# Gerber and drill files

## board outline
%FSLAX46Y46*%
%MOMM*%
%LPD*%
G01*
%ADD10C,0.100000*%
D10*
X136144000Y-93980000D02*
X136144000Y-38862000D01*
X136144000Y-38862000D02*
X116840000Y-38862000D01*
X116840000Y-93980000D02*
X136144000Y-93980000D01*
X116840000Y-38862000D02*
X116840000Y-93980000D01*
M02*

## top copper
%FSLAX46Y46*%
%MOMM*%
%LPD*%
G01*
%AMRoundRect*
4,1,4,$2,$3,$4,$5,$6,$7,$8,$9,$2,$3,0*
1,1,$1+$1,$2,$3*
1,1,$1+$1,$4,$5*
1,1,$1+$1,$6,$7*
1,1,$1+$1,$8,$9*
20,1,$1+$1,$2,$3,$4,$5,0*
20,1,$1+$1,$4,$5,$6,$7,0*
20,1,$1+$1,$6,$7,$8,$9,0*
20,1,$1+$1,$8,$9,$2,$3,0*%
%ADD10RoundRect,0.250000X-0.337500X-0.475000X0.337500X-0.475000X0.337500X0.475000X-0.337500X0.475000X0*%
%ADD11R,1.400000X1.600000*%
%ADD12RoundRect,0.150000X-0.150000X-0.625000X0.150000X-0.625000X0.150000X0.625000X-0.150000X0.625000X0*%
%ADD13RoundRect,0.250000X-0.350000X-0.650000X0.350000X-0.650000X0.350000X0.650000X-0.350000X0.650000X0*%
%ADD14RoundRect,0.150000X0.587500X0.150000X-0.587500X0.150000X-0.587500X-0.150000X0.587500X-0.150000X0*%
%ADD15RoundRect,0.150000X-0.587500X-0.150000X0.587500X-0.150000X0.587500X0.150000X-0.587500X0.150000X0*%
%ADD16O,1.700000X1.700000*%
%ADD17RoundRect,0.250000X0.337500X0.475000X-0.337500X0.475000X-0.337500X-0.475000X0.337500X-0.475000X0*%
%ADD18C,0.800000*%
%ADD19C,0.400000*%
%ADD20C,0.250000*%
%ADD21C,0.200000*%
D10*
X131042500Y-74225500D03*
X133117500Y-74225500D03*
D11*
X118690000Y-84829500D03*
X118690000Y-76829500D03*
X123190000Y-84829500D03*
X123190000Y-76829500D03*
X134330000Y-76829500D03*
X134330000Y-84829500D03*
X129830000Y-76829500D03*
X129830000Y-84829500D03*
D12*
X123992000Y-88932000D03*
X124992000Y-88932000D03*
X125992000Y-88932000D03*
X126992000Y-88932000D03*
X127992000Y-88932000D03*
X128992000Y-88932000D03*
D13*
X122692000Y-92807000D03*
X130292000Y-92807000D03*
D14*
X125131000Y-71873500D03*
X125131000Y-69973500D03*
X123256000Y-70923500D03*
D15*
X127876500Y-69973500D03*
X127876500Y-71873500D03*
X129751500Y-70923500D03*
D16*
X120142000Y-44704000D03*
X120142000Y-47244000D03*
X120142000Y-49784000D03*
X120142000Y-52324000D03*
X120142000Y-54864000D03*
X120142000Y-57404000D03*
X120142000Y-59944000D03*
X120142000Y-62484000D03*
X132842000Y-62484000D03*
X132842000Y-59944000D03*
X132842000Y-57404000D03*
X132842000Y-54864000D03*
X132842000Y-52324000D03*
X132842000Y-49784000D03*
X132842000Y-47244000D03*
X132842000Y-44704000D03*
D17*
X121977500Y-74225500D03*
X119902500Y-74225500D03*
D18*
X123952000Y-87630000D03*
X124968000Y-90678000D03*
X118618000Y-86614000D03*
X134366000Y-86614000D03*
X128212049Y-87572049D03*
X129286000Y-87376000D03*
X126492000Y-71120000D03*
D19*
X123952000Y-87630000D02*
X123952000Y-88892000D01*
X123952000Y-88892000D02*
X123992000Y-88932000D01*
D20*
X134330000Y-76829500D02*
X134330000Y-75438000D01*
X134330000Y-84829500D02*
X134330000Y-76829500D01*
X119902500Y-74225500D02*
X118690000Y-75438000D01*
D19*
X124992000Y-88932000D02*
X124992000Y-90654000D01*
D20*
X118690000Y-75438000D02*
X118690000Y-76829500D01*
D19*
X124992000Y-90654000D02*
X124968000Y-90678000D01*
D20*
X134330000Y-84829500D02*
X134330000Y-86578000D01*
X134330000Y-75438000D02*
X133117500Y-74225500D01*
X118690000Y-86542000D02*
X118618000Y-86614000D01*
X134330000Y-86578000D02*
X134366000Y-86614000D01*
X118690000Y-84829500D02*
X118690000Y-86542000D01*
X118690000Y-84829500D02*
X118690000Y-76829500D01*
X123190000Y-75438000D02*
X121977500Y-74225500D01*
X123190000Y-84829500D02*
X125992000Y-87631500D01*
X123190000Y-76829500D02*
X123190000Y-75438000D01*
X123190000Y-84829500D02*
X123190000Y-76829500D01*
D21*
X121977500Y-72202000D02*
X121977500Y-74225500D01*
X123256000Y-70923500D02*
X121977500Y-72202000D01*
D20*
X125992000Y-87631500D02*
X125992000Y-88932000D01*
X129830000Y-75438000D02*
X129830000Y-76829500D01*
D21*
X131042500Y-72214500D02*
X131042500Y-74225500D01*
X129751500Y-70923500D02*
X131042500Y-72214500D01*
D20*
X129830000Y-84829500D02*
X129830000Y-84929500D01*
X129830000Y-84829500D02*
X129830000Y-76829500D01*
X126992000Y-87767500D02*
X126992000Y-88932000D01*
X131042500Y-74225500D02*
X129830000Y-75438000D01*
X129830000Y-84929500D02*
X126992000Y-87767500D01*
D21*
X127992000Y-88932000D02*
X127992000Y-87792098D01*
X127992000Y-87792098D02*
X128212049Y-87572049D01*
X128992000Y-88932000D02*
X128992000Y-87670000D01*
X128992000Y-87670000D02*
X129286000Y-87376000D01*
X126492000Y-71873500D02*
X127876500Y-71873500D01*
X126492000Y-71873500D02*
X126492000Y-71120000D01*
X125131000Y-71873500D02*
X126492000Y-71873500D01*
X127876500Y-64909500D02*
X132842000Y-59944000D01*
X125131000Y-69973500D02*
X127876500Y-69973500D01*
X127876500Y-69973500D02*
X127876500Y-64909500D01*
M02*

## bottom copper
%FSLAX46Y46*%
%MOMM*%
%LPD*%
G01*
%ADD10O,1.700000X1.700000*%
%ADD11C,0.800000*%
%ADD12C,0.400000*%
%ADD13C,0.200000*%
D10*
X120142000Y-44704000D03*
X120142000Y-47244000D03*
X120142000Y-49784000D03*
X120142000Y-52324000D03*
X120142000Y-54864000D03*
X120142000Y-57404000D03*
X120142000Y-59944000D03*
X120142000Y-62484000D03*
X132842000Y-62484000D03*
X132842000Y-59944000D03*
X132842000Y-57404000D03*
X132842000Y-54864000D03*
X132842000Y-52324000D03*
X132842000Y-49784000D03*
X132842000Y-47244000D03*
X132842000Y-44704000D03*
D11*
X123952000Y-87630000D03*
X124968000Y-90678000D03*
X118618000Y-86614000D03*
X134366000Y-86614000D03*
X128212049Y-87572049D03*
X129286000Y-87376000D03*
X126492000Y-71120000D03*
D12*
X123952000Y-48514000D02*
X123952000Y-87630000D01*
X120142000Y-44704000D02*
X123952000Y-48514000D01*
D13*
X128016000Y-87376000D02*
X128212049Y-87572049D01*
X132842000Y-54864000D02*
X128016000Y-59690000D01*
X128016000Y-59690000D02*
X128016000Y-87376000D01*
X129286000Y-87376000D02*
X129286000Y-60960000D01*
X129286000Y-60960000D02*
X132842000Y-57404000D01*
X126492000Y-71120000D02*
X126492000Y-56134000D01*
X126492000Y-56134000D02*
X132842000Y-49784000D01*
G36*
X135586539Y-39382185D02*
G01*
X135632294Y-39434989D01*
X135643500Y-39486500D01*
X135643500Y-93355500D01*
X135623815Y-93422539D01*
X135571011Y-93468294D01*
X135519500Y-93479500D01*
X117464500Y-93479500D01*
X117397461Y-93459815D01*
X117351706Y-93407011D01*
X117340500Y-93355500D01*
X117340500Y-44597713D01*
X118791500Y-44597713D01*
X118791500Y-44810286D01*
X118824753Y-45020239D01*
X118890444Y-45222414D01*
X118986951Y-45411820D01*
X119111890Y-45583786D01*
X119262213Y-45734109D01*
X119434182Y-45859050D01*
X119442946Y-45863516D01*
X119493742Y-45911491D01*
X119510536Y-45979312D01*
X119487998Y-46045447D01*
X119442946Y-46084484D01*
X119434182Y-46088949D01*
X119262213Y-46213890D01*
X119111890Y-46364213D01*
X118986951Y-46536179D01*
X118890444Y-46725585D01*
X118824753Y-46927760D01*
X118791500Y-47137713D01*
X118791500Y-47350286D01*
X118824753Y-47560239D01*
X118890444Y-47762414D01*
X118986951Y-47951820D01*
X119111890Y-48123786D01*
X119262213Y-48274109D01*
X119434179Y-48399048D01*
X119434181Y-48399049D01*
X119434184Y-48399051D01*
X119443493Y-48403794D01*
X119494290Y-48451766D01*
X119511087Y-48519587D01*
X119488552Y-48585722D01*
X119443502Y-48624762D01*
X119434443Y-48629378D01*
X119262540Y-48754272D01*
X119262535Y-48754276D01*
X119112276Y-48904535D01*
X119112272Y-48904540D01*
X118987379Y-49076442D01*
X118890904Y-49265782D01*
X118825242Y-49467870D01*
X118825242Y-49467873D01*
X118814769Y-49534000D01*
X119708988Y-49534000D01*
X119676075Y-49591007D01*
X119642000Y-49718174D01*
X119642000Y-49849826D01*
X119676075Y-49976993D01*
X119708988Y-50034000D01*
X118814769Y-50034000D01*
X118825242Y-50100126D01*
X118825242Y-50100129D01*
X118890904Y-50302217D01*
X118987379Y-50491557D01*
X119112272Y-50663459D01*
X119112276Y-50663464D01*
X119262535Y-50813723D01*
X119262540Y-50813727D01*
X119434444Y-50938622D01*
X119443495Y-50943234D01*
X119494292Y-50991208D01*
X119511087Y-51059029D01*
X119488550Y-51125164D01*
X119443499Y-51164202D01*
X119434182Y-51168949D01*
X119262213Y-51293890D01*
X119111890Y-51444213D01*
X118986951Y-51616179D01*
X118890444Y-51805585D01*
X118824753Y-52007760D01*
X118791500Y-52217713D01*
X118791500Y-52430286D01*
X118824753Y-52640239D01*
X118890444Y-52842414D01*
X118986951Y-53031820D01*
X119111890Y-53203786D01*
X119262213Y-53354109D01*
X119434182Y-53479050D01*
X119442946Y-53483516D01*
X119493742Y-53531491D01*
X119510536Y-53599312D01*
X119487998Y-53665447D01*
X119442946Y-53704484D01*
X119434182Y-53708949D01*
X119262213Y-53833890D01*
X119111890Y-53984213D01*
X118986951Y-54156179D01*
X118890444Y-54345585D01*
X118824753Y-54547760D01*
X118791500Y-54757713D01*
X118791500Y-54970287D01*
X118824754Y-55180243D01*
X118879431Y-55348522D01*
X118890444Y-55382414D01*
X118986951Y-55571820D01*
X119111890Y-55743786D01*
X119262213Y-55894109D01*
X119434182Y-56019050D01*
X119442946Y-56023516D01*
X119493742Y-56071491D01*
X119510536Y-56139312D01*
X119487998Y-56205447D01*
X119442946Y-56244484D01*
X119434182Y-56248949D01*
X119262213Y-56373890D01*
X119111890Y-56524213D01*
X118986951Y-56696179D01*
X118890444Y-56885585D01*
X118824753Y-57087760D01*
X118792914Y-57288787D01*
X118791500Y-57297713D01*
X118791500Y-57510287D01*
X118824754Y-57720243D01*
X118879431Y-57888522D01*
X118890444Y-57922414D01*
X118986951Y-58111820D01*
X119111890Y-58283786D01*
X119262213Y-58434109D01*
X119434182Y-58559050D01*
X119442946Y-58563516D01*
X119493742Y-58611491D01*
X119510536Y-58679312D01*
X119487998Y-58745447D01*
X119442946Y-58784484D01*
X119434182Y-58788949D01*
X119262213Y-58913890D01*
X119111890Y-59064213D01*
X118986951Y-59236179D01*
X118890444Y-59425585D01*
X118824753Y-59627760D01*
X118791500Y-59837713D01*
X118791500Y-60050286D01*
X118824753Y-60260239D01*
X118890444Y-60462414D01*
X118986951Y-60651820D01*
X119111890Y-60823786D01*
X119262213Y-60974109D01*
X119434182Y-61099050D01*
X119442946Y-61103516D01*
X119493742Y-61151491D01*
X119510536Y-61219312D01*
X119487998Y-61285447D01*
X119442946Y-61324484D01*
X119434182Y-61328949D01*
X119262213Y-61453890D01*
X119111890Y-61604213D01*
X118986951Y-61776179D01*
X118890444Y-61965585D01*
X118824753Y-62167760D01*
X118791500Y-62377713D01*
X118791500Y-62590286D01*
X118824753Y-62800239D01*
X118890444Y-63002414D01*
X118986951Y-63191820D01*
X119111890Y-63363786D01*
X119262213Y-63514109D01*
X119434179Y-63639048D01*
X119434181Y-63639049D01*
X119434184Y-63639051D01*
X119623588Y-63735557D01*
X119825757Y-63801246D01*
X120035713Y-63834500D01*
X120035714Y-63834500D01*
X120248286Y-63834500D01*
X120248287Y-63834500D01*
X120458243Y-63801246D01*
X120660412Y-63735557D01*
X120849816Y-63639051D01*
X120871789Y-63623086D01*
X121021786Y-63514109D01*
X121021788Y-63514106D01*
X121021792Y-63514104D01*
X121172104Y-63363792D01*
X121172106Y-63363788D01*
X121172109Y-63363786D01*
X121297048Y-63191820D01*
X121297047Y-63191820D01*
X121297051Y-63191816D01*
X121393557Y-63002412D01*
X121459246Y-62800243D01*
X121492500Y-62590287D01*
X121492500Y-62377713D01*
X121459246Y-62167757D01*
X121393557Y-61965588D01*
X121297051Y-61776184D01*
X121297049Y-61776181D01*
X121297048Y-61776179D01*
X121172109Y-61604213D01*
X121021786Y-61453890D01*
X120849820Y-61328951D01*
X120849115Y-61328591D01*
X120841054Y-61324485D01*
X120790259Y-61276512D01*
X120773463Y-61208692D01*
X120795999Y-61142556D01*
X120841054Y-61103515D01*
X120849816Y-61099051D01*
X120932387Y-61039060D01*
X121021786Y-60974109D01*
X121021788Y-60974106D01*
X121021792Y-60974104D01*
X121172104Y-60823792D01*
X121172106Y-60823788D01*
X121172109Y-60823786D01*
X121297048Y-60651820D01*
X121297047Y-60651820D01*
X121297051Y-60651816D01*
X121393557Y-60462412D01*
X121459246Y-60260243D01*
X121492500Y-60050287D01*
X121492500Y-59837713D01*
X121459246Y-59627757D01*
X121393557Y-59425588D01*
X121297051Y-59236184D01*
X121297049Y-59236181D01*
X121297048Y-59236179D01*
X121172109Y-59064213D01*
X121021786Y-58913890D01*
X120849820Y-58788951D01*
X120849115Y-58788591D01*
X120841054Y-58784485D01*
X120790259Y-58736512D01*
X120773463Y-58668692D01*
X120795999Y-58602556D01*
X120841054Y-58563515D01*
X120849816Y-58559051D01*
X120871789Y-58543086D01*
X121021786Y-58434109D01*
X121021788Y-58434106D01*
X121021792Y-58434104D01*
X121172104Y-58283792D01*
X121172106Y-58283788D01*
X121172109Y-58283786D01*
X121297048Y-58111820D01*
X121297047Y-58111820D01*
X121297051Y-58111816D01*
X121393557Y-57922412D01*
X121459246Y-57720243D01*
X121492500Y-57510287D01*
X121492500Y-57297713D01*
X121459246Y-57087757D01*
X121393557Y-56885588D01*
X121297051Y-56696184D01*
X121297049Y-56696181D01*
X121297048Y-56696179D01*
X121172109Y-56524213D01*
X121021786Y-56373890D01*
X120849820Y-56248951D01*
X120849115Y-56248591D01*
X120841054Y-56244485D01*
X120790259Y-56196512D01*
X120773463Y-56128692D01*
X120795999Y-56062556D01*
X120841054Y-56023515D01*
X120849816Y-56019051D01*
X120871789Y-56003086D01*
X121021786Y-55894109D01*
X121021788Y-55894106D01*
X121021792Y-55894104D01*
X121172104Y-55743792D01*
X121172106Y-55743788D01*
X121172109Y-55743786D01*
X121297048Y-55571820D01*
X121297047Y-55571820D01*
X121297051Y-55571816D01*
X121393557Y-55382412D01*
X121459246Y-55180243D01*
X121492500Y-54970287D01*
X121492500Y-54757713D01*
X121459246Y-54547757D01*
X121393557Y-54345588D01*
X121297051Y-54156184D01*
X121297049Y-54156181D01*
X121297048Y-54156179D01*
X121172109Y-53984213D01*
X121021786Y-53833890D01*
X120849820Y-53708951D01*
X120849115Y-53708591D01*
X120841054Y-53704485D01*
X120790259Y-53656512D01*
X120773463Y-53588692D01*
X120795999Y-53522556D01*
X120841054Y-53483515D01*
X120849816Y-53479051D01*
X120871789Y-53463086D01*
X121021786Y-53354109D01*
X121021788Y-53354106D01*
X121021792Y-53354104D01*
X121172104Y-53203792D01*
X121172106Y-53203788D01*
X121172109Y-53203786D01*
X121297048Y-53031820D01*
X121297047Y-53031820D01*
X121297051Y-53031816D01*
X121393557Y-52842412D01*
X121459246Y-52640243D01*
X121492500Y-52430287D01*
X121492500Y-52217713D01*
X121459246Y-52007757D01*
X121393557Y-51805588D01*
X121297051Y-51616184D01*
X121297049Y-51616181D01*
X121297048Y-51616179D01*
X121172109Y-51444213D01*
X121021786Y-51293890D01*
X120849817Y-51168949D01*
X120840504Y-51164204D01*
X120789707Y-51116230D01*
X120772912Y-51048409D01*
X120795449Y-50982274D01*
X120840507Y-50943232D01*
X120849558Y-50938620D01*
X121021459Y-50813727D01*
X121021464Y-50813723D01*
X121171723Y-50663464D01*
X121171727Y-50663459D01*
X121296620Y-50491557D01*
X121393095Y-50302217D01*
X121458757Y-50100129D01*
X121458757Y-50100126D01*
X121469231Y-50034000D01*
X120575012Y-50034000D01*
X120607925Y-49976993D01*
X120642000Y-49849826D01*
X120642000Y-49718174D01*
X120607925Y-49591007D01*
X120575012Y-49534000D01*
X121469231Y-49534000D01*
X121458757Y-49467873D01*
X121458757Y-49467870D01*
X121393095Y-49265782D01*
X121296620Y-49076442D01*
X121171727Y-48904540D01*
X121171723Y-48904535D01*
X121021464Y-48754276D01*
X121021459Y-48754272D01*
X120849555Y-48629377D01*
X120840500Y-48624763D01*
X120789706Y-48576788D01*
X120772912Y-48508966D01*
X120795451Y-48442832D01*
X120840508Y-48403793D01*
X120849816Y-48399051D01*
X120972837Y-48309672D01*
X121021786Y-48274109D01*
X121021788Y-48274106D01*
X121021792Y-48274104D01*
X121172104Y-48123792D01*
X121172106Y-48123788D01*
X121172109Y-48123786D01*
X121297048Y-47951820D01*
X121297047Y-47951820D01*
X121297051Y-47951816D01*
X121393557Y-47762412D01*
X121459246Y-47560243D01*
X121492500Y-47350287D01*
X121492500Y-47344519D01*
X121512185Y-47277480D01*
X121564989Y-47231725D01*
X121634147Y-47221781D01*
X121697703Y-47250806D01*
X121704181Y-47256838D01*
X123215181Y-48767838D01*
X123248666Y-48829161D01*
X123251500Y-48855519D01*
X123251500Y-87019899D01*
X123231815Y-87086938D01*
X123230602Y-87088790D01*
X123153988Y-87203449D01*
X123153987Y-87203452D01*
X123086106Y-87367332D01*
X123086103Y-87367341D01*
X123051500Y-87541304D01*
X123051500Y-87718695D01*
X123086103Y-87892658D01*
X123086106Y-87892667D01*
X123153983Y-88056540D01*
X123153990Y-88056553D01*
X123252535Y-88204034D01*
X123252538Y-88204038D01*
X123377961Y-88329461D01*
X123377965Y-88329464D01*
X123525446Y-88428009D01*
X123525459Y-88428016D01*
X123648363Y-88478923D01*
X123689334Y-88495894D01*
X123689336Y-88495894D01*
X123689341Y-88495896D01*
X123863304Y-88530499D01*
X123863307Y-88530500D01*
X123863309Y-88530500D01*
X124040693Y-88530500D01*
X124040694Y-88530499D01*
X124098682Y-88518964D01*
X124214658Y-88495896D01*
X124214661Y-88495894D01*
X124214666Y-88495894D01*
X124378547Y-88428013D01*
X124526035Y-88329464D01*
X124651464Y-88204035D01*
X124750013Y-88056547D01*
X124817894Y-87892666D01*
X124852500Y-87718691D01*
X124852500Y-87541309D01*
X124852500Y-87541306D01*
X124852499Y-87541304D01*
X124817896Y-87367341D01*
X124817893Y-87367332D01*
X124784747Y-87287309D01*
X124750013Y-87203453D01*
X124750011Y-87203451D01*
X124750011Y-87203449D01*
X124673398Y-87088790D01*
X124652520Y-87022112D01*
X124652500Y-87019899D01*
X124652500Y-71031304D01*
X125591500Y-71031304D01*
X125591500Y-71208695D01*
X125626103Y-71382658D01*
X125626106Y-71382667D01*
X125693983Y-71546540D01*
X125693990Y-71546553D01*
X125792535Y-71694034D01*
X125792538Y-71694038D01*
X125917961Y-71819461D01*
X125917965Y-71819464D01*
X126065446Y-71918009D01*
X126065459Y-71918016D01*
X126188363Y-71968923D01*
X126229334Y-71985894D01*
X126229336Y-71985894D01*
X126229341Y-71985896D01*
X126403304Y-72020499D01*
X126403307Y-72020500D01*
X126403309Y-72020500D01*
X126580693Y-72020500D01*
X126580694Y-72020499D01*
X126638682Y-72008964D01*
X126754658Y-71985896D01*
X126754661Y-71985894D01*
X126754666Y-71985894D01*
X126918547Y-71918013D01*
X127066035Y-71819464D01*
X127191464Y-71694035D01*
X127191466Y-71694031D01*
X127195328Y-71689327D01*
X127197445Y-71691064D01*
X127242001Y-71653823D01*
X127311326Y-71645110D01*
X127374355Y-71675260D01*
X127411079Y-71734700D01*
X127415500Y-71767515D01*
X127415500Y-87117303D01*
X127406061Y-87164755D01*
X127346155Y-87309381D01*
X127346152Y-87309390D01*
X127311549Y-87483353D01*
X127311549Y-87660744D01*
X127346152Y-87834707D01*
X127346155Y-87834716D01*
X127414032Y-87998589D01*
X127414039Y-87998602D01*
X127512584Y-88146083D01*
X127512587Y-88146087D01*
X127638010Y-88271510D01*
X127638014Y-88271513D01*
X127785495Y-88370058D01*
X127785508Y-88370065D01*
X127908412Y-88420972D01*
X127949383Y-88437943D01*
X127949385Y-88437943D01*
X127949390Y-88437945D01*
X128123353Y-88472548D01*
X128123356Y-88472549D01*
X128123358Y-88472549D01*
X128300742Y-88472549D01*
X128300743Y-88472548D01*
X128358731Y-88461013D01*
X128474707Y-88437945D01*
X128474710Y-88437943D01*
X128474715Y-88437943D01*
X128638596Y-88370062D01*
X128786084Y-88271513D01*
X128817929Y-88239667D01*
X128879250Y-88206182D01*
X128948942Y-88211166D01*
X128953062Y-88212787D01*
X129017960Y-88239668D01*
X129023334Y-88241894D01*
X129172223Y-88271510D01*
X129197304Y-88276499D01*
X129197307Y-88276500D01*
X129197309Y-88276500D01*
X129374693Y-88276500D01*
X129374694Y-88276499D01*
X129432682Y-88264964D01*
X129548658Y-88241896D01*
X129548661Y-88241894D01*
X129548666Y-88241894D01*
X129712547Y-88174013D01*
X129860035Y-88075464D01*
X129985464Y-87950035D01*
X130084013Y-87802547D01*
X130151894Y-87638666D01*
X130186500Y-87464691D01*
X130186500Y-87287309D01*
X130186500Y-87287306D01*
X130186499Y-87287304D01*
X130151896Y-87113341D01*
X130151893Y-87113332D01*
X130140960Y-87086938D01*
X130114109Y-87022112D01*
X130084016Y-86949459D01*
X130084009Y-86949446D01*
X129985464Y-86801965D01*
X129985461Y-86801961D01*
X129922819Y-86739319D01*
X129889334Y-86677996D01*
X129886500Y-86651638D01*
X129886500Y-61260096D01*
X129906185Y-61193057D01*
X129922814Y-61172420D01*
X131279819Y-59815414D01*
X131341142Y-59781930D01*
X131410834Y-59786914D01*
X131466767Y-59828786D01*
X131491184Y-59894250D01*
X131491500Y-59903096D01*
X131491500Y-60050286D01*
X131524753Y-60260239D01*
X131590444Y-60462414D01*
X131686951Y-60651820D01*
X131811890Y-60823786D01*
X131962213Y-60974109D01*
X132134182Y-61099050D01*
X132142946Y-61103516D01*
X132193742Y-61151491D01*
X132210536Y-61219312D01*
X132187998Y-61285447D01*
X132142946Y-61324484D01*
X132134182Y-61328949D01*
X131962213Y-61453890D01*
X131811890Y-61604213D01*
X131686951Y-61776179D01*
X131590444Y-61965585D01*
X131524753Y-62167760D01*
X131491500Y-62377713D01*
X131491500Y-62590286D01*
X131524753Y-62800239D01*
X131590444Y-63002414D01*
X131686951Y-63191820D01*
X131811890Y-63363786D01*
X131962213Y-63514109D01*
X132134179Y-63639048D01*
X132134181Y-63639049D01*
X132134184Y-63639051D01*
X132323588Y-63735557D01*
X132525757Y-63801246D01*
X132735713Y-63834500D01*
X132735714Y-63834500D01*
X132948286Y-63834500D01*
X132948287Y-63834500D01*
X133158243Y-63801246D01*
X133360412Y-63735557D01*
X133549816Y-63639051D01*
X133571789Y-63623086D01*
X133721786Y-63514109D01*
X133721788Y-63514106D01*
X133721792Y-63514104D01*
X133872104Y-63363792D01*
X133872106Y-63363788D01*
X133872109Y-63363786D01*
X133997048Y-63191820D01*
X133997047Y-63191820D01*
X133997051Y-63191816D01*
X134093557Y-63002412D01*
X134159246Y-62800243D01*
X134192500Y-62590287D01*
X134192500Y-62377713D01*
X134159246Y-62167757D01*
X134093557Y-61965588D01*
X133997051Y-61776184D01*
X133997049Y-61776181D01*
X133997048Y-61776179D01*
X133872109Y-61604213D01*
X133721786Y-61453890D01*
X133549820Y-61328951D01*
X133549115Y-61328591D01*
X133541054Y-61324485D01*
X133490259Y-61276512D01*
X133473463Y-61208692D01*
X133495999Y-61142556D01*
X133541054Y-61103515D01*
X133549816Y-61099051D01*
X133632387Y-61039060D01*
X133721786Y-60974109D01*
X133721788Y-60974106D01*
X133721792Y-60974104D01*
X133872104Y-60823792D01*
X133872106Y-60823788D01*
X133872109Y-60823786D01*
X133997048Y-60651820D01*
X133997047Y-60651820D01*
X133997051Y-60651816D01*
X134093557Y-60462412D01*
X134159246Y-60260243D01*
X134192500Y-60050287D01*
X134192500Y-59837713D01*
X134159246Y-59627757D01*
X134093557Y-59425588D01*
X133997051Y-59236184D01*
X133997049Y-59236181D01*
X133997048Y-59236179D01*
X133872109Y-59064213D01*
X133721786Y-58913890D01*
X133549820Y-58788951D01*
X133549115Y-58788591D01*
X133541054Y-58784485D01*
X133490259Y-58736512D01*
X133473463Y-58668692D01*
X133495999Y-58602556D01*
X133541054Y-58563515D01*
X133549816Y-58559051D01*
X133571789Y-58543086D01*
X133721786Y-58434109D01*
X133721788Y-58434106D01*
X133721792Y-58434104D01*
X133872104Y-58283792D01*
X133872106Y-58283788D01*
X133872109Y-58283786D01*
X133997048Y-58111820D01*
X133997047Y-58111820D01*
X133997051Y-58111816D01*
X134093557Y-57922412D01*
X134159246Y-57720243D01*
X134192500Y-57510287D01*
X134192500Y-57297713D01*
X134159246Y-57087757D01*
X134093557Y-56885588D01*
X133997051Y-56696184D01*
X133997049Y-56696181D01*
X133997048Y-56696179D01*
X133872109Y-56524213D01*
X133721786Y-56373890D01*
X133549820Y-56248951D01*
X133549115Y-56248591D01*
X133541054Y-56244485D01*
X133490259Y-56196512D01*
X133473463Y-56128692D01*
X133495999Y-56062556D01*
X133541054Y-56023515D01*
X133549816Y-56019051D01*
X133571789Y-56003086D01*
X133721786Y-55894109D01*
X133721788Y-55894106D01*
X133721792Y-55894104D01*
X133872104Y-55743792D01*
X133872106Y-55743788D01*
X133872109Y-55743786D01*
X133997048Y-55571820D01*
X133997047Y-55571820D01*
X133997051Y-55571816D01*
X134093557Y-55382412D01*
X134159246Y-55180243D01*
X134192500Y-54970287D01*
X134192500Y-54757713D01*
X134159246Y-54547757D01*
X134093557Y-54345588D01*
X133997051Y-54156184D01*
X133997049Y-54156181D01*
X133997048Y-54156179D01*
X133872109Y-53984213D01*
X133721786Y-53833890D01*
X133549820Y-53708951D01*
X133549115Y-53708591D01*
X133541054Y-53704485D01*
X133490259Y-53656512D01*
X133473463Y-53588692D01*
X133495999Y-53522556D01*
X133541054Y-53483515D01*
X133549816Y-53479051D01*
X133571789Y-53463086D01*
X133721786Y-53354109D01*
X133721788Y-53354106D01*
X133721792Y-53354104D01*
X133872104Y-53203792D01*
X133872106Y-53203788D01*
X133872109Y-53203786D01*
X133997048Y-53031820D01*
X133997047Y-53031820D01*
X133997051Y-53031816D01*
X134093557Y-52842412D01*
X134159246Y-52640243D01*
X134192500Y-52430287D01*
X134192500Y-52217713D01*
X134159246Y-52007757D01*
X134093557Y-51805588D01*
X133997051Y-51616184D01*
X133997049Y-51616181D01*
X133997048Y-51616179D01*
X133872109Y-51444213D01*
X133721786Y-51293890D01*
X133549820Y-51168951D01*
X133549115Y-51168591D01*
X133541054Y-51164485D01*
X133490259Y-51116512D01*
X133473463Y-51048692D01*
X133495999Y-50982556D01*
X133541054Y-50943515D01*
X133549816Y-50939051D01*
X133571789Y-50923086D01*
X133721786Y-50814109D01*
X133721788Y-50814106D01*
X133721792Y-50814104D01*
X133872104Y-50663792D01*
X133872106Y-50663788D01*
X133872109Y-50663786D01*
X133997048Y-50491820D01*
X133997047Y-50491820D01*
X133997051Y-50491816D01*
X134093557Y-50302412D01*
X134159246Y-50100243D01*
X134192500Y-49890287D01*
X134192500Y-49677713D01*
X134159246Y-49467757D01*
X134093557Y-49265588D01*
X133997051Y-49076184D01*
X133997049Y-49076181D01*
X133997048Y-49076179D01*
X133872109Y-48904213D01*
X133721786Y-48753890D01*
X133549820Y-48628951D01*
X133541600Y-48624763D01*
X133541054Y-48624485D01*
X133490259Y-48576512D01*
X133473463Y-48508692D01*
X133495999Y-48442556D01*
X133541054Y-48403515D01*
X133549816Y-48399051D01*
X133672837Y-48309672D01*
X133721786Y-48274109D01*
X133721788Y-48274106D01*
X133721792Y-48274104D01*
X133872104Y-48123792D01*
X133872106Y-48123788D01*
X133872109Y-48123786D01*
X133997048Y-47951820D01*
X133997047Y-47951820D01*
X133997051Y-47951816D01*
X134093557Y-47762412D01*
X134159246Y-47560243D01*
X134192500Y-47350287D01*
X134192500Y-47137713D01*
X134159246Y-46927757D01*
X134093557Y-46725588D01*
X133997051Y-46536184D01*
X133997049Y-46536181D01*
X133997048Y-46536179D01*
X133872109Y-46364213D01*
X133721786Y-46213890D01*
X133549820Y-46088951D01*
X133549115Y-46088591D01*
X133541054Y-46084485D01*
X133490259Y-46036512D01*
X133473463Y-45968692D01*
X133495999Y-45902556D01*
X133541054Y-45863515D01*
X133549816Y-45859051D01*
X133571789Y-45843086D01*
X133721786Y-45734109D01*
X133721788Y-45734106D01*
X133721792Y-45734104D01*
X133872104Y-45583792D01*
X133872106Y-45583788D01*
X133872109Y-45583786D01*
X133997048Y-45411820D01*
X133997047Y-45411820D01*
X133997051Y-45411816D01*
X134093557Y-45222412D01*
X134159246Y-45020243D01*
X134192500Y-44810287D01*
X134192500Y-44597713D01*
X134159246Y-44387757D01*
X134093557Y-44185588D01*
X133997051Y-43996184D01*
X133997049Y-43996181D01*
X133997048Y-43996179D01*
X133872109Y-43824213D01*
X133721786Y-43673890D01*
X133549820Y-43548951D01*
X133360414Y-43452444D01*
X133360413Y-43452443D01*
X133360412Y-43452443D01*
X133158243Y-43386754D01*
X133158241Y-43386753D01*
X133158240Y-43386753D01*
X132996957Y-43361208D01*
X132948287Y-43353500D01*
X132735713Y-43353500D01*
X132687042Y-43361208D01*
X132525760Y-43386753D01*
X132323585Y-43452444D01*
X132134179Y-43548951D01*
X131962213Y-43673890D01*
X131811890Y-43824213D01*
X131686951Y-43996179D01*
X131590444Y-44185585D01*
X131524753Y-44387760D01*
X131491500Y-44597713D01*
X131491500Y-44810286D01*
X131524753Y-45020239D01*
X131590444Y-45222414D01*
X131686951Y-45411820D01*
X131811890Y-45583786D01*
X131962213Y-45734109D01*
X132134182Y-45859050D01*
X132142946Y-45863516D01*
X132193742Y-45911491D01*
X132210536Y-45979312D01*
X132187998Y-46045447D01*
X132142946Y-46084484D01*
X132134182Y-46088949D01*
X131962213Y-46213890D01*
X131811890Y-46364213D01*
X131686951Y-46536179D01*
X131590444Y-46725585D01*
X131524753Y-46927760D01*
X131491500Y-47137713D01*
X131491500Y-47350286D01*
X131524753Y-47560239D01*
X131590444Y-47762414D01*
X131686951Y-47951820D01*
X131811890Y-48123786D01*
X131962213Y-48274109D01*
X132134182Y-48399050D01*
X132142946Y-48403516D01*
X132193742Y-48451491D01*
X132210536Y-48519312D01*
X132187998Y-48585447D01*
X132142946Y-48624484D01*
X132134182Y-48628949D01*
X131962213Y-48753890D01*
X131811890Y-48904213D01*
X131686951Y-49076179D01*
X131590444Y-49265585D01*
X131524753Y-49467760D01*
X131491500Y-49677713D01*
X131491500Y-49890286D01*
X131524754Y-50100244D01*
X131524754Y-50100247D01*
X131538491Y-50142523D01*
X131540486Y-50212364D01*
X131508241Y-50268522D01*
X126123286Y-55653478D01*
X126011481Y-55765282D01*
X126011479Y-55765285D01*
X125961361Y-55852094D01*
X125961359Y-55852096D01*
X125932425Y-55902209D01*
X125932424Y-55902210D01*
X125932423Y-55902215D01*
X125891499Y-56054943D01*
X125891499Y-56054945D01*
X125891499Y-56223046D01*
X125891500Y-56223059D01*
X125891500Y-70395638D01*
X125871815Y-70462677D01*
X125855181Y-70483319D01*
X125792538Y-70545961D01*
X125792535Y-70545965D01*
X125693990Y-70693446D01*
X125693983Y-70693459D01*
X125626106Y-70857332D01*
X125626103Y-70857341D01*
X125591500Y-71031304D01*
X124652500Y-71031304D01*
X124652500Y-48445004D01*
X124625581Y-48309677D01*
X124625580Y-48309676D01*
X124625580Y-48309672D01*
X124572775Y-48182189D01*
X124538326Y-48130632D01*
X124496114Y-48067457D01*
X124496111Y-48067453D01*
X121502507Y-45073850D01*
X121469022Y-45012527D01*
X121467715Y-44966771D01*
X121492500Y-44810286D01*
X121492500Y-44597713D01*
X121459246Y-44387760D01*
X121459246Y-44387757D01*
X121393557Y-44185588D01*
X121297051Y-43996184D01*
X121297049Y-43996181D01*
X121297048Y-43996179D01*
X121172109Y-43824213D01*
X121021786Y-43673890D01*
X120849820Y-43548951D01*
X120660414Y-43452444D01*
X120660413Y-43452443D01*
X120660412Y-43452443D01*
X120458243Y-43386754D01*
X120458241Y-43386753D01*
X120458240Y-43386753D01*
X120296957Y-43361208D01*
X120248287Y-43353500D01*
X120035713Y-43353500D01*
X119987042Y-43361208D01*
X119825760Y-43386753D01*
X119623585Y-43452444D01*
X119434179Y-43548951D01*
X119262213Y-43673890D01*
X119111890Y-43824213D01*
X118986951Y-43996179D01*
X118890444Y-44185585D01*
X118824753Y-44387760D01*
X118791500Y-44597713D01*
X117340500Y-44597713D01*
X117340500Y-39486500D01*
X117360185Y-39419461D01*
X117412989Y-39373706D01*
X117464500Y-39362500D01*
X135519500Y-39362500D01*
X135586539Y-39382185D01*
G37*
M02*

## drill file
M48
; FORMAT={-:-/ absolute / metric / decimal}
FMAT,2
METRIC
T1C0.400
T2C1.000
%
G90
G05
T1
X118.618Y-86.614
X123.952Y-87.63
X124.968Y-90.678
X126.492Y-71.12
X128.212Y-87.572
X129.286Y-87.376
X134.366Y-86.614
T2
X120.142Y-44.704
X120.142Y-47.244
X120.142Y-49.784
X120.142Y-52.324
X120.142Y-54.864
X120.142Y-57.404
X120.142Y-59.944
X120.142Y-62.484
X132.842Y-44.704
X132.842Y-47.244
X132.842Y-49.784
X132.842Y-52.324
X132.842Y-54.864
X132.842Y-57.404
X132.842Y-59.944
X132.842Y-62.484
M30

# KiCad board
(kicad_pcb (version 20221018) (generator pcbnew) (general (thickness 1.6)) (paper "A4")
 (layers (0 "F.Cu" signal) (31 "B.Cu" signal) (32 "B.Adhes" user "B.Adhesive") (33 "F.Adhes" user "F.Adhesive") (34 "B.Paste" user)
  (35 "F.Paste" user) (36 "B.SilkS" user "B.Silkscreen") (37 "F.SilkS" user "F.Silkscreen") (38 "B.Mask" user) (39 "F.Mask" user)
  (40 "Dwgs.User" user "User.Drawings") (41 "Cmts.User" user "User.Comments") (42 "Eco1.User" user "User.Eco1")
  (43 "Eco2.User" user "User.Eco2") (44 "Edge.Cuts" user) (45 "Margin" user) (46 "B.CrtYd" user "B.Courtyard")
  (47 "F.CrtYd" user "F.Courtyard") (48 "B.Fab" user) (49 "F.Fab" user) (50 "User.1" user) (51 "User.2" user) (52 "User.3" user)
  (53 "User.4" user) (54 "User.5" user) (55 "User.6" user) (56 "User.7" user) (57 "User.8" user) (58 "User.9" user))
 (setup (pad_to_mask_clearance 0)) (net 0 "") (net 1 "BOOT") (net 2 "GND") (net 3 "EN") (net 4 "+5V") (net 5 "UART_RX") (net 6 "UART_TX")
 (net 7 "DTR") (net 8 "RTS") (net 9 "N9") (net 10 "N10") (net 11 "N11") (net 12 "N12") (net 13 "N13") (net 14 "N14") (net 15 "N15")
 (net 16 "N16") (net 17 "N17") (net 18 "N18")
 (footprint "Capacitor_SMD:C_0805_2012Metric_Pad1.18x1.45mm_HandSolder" (layer "F.Cu") (at 132.08 74.2255)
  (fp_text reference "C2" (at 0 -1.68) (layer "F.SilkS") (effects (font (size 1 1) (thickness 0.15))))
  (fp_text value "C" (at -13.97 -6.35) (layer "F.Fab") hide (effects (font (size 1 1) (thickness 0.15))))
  (pad "1" smd roundrect (at -1.0375 0) (size 1.175 1.45) (layers "F.Cu" "F.Paste" "F.Mask") (roundrect_rratio 0.2127659574) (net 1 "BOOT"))
  (pad "2" smd roundrect (at 1.0375 0) (size 1.175 1.45) (layers "F.Cu" "F.Paste" "F.Mask") (roundrect_rratio 0.2127659574) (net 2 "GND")))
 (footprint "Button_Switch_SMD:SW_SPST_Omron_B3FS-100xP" (layer "F.Cu") (at 120.94 80.8295 90)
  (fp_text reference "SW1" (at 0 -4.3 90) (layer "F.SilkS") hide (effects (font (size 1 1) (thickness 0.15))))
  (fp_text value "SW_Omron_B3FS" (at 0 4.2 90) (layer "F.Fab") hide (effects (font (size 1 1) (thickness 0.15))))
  (pad "1" smd rect (at -4 -2.25 270) (size 1.6 1.4) (layers "F.Cu" "F.Paste" "F.Mask") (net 2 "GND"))
  (pad "1" smd rect (at 4 -2.25 270) (size 1.6 1.4) (layers "F.Cu" "F.Paste" "F.Mask") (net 2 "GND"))
  (pad "2" smd rect (at -4 2.25 270) (size 1.6 1.4) (layers "F.Cu" "F.Paste" "F.Mask") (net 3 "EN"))
  (pad "2" smd rect (at 4 2.25 270) (size 1.6 1.4) (layers "F.Cu" "F.Paste" "F.Mask") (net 3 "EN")))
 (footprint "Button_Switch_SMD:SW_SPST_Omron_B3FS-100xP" (layer "F.Cu") (at 132.08 80.8295 -90)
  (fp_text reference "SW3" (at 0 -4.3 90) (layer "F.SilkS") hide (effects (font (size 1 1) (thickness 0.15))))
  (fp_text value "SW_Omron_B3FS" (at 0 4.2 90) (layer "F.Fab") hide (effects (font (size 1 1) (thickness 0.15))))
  (pad "1" smd rect (at -4 -2.25 90) (size 1.6 1.4) (layers "F.Cu" "F.Paste" "F.Mask") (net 2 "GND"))
  (pad "1" smd rect (at 4 -2.25 90) (size 1.6 1.4) (layers "F.Cu" "F.Paste" "F.Mask") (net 2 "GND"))
  (pad "2" smd rect (at -4 2.25 90) (size 1.6 1.4) (layers "F.Cu" "F.Paste" "F.Mask") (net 1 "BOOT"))
  (pad "2" smd rect (at 4 2.25 90) (size 1.6 1.4) (layers "F.Cu" "F.Paste" "F.Mask") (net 1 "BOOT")))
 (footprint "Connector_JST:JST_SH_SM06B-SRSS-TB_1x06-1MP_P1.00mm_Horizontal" (layer "F.Cu") (at 126.492 90.932)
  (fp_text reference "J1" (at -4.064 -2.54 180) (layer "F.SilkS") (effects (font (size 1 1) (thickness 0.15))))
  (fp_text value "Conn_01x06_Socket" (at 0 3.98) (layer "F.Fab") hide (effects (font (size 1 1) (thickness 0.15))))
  (pad "1" smd roundrect (at -2.5 -2) (size 0.6 1.55) (layers "F.Cu" "F.Paste" "F.Mask") (roundrect_rratio 0.25) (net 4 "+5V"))
  (pad "2" smd roundrect (at -1.5 -2) (size 0.6 1.55) (layers "F.Cu" "F.Paste" "F.Mask") (roundrect_rratio 0.25) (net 2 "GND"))
  (pad "3" smd roundrect (at -0.5 -2) (size 0.6 1.55) (layers "F.Cu" "F.Paste" "F.Mask") (roundrect_rratio 0.25) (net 3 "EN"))
  (pad "4" smd roundrect (at 0.5 -2) (size 0.6 1.55) (layers "F.Cu" "F.Paste" "F.Mask") (roundrect_rratio 0.25) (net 1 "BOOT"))
  (pad "5" smd roundrect (at 1.5 -2) (size 0.6 1.55) (layers "F.Cu" "F.Paste" "F.Mask") (roundrect_rratio 0.25) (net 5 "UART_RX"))
  (pad "6" smd roundrect (at 2.5 -2) (size 0.6 1.55) (layers "F.Cu" "F.Paste" "F.Mask") (roundrect_rratio 0.25) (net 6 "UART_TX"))
  (pad "MP" smd roundrect (at -3.8 1.875) (size 1.2 1.8) (layers "F.Cu" "F.Paste" "F.Mask") (roundrect_rratio 0.2083333333))
  (pad "MP" smd roundrect (at 3.8 1.875) (size 1.2 1.8) (layers "F.Cu" "F.Paste" "F.Mask") (roundrect_rratio 0.2083333333)))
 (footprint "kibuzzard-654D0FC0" (layer "F.Cu") (at 120.904 86.868)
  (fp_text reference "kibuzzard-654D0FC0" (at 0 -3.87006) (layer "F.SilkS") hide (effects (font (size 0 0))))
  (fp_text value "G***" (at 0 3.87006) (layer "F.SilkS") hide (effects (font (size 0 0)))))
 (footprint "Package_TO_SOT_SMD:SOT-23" (layer "F.Cu") (at 124.1935 70.9235 180)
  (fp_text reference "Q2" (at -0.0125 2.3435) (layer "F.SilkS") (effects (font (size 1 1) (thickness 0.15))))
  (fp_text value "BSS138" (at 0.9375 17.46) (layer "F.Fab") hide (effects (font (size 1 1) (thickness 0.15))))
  (pad "1" smd roundrect (at -0.9375 -0.95 180) (size 1.475 0.6) (layers "F.Cu" "F.Paste" "F.Mask") (roundrect_rratio 0.25) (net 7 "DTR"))
  (pad "2" smd roundrect (at -0.9375 0.95 180) (size 1.475 0.6) (layers "F.Cu" "F.Paste" "F.Mask") (roundrect_rratio 0.25) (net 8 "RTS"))
  (pad "3" smd roundrect (at 0.9375 0 180) (size 1.475 0.6) (layers "F.Cu" "F.Paste" "F.Mask") (roundrect_rratio 0.25) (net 3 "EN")))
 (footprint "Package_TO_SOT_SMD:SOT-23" (layer "F.Cu") (at 128.814 70.9235)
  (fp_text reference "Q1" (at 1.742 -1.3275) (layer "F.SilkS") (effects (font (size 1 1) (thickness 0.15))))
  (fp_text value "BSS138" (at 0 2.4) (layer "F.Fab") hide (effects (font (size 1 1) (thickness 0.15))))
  (pad "1" smd roundrect (at -0.9375 -0.95) (size 1.475 0.6) (layers "F.Cu" "F.Paste" "F.Mask") (roundrect_rratio 0.25) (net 8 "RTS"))
  (pad "2" smd roundrect (at -0.9375 0.95) (size 1.475 0.6) (layers "F.Cu" "F.Paste" "F.Mask") (roundrect_rratio 0.25) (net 7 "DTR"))
  (pad "3" smd roundrect (at 0.9375 0) (size 1.475 0.6) (layers "F.Cu" "F.Paste" "F.Mask") (roundrect_rratio 0.25) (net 1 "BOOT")))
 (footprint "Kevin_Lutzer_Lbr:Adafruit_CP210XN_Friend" (layer "F.Cu") (at 126.492 53.594)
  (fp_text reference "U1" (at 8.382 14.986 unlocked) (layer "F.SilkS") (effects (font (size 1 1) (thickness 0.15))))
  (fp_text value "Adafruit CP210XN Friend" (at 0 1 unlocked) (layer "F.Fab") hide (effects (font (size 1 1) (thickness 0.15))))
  (pad "1" thru_hole oval (at -6.35 -8.89) (size 1.7 1.7) (drill 1) (layers "*.Cu" "*.Mask") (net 4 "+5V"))
  (pad "2" thru_hole oval (at -6.35 -6.35) (size 1.7 1.7) (drill 1) (layers "*.Cu" "*.Mask") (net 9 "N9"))
  (pad "3" thru_hole oval (at -6.35 -3.81) (size 1.7 1.7) (drill 1) (layers "*.Cu" "*.Mask") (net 2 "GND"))
  (pad "4" thru_hole oval (at -6.35 -1.27) (size 1.7 1.7) (drill 1) (layers "*.Cu" "*.Mask") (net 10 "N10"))
  (pad "5" thru_hole oval (at -6.35 1.27) (size 1.7 1.7) (drill 1) (layers "*.Cu" "*.Mask") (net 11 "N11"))
  (pad "6" thru_hole oval (at -6.35 3.81) (size 1.7 1.7) (drill 1) (layers "*.Cu" "*.Mask") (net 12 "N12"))
  (pad "7" thru_hole oval (at -6.35 6.35) (size 1.7 1.7) (drill 1) (layers "*.Cu" "*.Mask") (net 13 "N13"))
  (pad "8" thru_hole oval (at -6.35 8.89) (size 1.7 1.7) (drill 1) (layers "*.Cu" "*.Mask") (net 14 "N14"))
  (pad "9" thru_hole oval (at 6.35 8.89) (size 1.7 1.7) (drill 1) (layers "*.Cu" "*.Mask") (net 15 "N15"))
  (pad "10" thru_hole oval (at 6.35 6.35) (size 1.7 1.7) (drill 1) (layers "*.Cu" "*.Mask") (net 8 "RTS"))
  (pad "11" thru_hole oval (at 6.35 3.81) (size 1.7 1.7) (drill 1) (layers "*.Cu" "*.Mask") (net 6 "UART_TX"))
  (pad "12" thru_hole oval (at 6.35 1.27) (size 1.7 1.7) (drill 1) (layers "*.Cu" "*.Mask") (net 5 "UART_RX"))
  (pad "13" thru_hole oval (at 6.35 -1.27) (size 1.7 1.7) (drill 1) (layers "*.Cu" "*.Mask") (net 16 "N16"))
  (pad "14" thru_hole oval (at 6.35 -3.81) (size 1.7 1.7) (drill 1) (layers "*.Cu" "*.Mask") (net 7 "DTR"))
  (pad "15" thru_hole oval (at 6.35 -6.35) (size 1.7 1.7) (drill 1) (layers "*.Cu" "*.Mask") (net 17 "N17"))
  (pad "16" thru_hole oval (at 6.35 -8.89) (size 1.7 1.7) (drill 1) (layers "*.Cu" "*.Mask") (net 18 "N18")))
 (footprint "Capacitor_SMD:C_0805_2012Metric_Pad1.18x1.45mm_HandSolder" (layer "F.Cu") (at 120.94 74.2255 180)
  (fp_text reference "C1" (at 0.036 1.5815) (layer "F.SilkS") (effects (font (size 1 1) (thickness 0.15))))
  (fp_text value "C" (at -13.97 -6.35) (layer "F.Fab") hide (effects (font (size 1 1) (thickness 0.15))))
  (pad "1" smd roundrect (at -1.0375 0 180) (size 1.175 1.45) (layers "F.Cu" "F.Paste" "F.Mask") (roundrect_rratio 0.2127659574)
   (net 3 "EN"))
  (pad "2" smd roundrect (at 1.0375 0 180) (size 1.175 1.45) (layers "F.Cu" "F.Paste" "F.Mask") (roundrect_rratio 0.2127659574)
   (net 2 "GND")))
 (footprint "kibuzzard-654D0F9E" (layer "F.Cu") (at 132.08 86.868)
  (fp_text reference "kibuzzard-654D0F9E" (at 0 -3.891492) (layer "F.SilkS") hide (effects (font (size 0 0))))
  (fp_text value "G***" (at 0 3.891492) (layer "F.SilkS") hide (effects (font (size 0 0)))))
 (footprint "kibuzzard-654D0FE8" (layer "B.Cu") (at 118.364 73.66 -90)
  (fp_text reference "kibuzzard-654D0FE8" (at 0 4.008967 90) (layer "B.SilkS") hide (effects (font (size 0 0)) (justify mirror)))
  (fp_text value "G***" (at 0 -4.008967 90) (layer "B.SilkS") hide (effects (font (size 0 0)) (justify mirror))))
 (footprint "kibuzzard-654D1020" (layer "B.Cu") (at 120.396 70.104 -90)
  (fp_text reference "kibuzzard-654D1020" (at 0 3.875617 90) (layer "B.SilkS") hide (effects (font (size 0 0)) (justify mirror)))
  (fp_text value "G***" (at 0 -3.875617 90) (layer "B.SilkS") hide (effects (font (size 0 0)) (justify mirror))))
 (gr_line (start 136.144 93.98) (end 136.144 38.862) (stroke (width 0.1) (type default)) (layer "Edge.Cuts"))
 (gr_line (start 136.144 38.862) (end 116.84 38.862) (stroke (width 0.1) (type default)) (layer "Edge.Cuts"))
 (gr_line (start 116.84 93.98) (end 136.144 93.98) (stroke (width 0.1) (type default)) (layer "Edge.Cuts"))
 (gr_line (start 116.84 38.862) (end 116.84 93.98) (stroke (width 0.1) (type default)) (layer "Edge.Cuts"))
 (segment (start 123.952 87.63) (end 123.952 88.892) (width 0.4) (layer "F.Cu") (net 4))
 (segment (start 123.952 88.892) (end 123.992 88.932) (width 0.4) (layer "F.Cu") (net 4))
 (via (at 123.952 87.63) (size 0.8) (drill 0.4) (layers "F.Cu" "B.Cu") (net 4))
 (segment (start 123.952 48.514) (end 123.952 87.63) (width 0.4) (layer "B.Cu") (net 4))
 (segment (start 120.142 44.704) (end 123.952 48.514) (width 0.4) (layer "B.Cu") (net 4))
 (segment (start 134.33 76.8295) (end 134.33 75.438) (width 0.25) (layer "F.Cu") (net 2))
 (segment (start 134.33 84.8295) (end 134.33 76.8295) (width 0.25) (layer "F.Cu") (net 2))
 (segment (start 119.9025 74.2255) (end 118.69 75.438) (width 0.25) (layer "F.Cu") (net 2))
 (segment (start 124.992 88.932) (end 124.992 90.654) (width 0.4) (layer "F.Cu") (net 2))
 (segment (start 118.69 75.438) (end 118.69 76.8295) (width 0.25) (layer "F.Cu") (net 2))
 (segment (start 124.992 90.654) (end 124.968 90.678) (width 0.4) (layer "F.Cu") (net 2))
 (segment (start 134.33 84.8295) (end 134.33 86.578) (width 0.25) (layer "F.Cu") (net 2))
 (segment (start 134.33 75.438) (end 133.1175 74.2255) (width 0.25) (layer "F.Cu") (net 2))
 (segment (start 118.69 86.542) (end 118.618 86.614) (width 0.25) (layer "F.Cu") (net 2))
 (segment (start 134.33 86.578) (end 134.366 86.614) (width 0.25) (layer "F.Cu") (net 2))
 (segment (start 118.69 84.8295) (end 118.69 86.542) (width 0.25) (layer "F.Cu") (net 2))
 (segment (start 118.69 84.8295) (end 118.69 76.8295) (width 0.25) (layer "F.Cu") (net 2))
 (via (at 124.968 90.678) (size 0.8) (drill 0.4) (layers "F.Cu" "B.Cu") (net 2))
 (via (at 118.618 86.614) (size 0.8) (drill 0.4) (layers "F.Cu" "B.Cu") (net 2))
 (via (at 134.366 86.614) (size 0.8) (drill 0.4) (layers "F.Cu" "B.Cu") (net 2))
 (segment (start 123.19 75.438) (end 121.9775 74.2255) (width 0.25) (layer "F.Cu") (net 3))
 (segment (start 123.19 84.8295) (end 125.992 87.6315) (width 0.25) (layer "F.Cu") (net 3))
 (segment (start 123.19 76.8295) (end 123.19 75.438) (width 0.25) (layer "F.Cu") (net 3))
 (segment (start 123.19 84.8295) (end 123.19 76.8295) (width 0.25) (layer "F.Cu") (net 3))
 (segment (start 121.9775 72.202) (end 121.9775 74.2255) (width 0.2) (layer "F.Cu") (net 3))
 (segment (start 123.256 70.9235) (end 121.9775 72.202) (width 0.2) (layer "F.Cu") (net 3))
 (segment (start 125.992 87.6315) (end 125.992 88.932) (width 0.25) (layer "F.Cu") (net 3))
 (segment (start 129.83 75.438) (end 129.83 76.8295) (width 0.25) (layer "F.Cu") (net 1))
 (segment (start 131.0425 72.2145) (end 131.0425 74.2255) (width 0.2) (layer "F.Cu") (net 1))
 (segment (start 129.7515 70.9235) (end 131.0425 72.2145) (width 0.2) (layer "F.Cu") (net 1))
 (segment (start 129.83 84.8295) (end 129.83 84.9295) (width 0.25) (layer "F.Cu") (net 1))
 (segment (start 129.83 84.8295) (end 129.83 76.8295) (width 0.25) (layer "F.Cu") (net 1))
 (segment (start 126.992 87.7675) (end 126.992 88.932) (width 0.25) (layer "F.Cu") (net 1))
 (segment (start 131.0425 74.2255) (end 129.83 75.438) (width 0.25) (layer "F.Cu") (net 1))
 (segment (start 129.83 84.9295) (end 126.992 87.7675) (width 0.25) (layer "F.Cu") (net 1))
 (segment (start 127.992 88.932) (end 127.992 87.792098) (width 0.2) (layer "F.Cu") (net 5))
 (segment (start 127.992 87.792098) (end 128.212049 87.572049) (width 0.2) (layer "F.Cu") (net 5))
 (via (at 128.212049 87.572049) (size 0.8) (drill 0.4) (layers "F.Cu" "B.Cu") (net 5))
 (segment (start 128.016 87.376) (end 128.212049 87.572049) (width 0.2) (layer "B.Cu") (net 5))
 (segment (start 132.842 54.864) (end 128.016 59.69) (width 0.2) (layer "B.Cu") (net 5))
 (segment (start 128.016 59.69) (end 128.016 87.376) (width 0.2) (layer "B.Cu") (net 5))
 (segment (start 128.992 88.932) (end 128.992 87.67) (width 0.2) (layer "F.Cu") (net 6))
 (segment (start 128.992 87.67) (end 129.286 87.376) (width 0.2) (layer "F.Cu") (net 6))
 (via (at 129.286 87.376) (size 0.8) (drill 0.4) (layers "F.Cu" "B.Cu") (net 6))
 (segment (start 129.286 87.376) (end 129.286 60.96) (width 0.2) (layer "B.Cu") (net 6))
 (segment (start 129.286 60.96) (end 132.842 57.404) (width 0.2) (layer "B.Cu") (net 6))
 (segment (start 126.492 71.8735) (end 127.8765 71.8735) (width 0.2) (layer "F.Cu") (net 7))
 (segment (start 126.492 71.8735) (end 126.492 71.12) (width 0.2) (layer "F.Cu") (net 7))
 (segment (start 125.131 71.8735) (end 126.492 71.8735) (width 0.2) (layer "F.Cu") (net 7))
 (via (at 126.492 71.12) (size 0.8) (drill 0.4) (layers "F.Cu" "B.Cu") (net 7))
 (segment (start 126.492 71.12) (end 126.492 56.134) (width 0.2) (layer "B.Cu") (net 7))
 (segment (start 126.492 56.134) (end 132.842 49.784) (width 0.2) (layer "B.Cu") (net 7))
 (segment (start 127.8765 64.9095) (end 132.842 59.944) (width 0.2) (layer "F.Cu") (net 8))
 (segment (start 125.131 69.9735) (end 127.8765 69.9735) (width 0.2) (layer "F.Cu") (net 8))
 (segment (start 127.8765 69.9735) (end 127.8765 64.9095) (width 0.2) (layer "F.Cu") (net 8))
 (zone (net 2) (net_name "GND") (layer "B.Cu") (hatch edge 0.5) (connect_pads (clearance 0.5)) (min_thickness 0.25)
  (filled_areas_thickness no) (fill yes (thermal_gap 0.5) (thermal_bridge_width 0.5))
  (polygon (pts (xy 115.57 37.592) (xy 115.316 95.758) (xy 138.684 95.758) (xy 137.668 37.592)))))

